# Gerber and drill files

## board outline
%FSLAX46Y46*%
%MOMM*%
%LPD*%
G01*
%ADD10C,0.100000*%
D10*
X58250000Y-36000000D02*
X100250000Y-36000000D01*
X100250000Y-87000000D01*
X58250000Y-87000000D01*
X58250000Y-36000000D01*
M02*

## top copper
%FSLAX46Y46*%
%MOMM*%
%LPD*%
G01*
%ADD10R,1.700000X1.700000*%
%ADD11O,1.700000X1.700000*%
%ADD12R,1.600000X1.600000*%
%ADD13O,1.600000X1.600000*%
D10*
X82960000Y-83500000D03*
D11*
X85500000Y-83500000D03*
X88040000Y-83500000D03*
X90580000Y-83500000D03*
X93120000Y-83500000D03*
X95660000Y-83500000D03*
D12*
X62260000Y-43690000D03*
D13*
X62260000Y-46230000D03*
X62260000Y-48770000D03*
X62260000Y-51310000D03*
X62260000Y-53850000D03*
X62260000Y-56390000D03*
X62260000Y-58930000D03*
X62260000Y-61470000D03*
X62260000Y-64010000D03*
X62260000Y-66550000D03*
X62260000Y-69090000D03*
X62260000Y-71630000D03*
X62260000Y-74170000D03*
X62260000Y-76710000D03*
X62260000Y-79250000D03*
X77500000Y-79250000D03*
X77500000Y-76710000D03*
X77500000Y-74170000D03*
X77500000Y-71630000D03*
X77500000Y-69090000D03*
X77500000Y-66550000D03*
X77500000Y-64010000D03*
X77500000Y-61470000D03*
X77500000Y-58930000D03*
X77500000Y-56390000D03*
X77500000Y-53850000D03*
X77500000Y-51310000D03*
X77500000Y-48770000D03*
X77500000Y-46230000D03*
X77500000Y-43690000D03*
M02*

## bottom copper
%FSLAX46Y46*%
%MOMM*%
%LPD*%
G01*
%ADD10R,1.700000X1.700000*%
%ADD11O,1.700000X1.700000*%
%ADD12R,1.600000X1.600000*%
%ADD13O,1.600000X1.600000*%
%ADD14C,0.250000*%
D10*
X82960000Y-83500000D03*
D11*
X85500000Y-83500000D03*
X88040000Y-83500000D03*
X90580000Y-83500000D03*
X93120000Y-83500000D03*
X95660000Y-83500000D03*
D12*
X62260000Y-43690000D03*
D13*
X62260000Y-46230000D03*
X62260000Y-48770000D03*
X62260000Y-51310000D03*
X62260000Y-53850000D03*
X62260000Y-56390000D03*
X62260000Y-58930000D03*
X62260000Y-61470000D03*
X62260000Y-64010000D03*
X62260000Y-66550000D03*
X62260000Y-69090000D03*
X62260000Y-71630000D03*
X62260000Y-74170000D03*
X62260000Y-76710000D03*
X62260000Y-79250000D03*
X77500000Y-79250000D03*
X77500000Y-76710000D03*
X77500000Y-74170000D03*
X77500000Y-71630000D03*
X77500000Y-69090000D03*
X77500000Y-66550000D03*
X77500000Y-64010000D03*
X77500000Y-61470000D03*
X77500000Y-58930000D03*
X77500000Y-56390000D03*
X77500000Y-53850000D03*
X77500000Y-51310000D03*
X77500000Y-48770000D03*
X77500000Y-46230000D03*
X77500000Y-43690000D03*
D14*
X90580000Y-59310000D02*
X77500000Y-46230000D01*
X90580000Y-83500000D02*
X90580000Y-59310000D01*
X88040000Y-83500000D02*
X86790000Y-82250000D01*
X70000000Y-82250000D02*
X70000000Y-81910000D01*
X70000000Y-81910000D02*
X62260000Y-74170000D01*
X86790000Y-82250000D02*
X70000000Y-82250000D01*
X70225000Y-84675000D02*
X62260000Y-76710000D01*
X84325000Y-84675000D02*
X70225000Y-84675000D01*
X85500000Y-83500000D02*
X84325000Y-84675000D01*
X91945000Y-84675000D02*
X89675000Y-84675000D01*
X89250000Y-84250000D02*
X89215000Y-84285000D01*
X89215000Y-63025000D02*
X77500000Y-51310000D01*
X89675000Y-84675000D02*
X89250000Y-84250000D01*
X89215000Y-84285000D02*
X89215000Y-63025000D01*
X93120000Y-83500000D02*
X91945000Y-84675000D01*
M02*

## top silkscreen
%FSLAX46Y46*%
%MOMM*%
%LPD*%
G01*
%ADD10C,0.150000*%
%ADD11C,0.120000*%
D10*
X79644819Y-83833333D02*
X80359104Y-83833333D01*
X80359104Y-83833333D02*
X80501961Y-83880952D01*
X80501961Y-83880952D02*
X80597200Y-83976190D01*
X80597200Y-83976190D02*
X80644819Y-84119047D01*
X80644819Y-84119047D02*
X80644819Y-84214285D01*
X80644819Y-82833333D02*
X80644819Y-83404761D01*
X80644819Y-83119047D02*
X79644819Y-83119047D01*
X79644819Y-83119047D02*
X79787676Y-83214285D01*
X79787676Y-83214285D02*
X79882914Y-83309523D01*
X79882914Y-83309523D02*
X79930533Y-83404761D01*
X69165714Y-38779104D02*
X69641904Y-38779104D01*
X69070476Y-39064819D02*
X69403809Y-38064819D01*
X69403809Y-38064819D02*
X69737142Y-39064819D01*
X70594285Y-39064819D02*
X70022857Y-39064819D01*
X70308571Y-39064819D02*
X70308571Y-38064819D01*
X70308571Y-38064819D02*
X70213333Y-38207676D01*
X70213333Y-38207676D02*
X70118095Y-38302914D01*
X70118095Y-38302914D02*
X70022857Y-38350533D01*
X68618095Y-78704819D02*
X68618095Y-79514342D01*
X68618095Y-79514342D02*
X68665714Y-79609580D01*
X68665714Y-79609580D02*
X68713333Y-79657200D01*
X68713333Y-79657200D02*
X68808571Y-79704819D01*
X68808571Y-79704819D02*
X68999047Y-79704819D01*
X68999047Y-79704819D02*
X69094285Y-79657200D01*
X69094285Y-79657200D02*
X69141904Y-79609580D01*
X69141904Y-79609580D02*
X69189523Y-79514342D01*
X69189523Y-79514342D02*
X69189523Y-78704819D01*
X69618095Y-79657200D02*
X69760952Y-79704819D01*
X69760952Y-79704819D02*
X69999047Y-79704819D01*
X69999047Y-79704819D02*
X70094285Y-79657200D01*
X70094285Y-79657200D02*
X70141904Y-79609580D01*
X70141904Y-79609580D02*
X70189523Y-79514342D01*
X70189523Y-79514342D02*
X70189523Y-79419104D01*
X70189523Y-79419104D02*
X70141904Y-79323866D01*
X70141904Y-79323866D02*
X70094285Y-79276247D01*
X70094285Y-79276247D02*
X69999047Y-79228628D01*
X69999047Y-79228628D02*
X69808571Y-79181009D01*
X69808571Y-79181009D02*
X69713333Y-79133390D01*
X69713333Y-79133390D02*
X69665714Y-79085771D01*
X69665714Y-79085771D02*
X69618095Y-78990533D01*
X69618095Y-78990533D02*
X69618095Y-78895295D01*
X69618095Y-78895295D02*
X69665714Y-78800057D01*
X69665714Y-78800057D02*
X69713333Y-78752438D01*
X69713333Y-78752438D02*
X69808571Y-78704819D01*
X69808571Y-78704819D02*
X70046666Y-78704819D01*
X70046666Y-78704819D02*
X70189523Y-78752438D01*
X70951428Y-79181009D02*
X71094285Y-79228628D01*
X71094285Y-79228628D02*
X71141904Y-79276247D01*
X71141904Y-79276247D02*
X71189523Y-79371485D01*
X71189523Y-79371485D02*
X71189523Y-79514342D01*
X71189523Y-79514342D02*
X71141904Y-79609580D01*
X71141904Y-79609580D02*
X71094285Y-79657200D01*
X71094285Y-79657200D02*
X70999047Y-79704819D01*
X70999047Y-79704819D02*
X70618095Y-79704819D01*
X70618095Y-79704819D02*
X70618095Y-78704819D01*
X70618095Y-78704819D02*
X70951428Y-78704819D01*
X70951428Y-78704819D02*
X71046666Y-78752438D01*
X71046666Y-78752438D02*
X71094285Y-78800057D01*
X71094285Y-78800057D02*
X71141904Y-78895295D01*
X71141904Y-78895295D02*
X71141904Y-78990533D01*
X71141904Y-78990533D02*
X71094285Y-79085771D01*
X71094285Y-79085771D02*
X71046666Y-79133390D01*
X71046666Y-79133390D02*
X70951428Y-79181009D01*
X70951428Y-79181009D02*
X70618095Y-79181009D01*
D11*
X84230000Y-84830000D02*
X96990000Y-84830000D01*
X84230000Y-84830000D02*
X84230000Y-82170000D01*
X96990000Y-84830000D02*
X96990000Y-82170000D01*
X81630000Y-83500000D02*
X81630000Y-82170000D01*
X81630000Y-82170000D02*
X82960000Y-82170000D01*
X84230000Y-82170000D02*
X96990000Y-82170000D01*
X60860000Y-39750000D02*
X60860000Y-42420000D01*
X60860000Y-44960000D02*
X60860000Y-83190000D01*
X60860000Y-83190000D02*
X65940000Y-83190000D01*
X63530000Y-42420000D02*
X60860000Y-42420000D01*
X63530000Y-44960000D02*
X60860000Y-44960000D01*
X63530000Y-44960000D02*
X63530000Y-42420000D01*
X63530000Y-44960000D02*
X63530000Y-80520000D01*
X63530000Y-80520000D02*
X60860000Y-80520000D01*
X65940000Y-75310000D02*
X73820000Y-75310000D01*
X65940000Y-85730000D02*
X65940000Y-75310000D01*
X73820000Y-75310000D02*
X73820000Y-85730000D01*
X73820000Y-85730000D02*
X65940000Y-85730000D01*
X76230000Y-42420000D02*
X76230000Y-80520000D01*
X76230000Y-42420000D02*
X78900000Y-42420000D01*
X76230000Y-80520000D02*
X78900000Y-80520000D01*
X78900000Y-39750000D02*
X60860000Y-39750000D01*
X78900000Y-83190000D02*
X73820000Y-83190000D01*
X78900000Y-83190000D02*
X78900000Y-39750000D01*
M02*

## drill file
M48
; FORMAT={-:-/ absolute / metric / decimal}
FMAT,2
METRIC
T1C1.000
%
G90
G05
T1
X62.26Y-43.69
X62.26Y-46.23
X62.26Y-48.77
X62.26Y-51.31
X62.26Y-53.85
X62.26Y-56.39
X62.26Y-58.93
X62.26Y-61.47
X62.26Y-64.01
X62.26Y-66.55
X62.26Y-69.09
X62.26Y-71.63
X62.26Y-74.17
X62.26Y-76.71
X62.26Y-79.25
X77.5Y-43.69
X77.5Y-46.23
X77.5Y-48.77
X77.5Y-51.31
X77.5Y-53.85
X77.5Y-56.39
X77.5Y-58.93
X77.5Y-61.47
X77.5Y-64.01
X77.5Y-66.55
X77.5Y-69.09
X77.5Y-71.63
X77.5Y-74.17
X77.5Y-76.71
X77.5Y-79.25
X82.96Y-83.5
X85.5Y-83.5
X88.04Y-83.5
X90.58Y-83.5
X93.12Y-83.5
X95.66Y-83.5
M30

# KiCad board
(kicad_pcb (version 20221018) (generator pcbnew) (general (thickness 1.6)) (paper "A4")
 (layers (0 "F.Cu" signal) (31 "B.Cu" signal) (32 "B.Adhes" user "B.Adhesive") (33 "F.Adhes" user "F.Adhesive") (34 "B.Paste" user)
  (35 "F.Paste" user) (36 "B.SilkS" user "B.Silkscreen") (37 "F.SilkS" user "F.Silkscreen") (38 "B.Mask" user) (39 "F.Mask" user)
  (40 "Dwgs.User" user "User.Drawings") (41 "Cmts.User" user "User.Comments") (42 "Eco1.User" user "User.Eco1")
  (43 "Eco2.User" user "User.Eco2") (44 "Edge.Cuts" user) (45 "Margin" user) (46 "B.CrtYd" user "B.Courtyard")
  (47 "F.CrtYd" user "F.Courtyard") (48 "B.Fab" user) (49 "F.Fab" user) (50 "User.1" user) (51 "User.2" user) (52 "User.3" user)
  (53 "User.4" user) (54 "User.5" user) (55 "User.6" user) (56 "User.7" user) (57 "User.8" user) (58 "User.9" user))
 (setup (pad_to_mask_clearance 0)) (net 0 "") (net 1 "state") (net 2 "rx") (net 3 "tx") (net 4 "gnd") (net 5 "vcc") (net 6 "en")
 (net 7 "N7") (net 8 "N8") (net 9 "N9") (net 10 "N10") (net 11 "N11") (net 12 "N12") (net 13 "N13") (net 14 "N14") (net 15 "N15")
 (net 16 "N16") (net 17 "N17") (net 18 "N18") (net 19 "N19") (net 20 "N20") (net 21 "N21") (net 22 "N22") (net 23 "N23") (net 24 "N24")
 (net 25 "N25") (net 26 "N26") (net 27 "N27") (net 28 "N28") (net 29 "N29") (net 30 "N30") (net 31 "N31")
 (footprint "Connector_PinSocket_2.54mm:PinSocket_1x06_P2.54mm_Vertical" (layer "F.Cu") (at 82.96 83.5 90)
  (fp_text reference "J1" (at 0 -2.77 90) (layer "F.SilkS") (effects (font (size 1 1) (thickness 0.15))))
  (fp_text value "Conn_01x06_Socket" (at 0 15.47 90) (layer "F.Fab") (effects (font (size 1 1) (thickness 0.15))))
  (fp_line (start -1.33 1.27) (end -1.33 14.03) (stroke (width 0.12) (type solid)) (layer "F.SilkS"))
  (fp_line (start -1.33 1.27) (end 1.33 1.27) (stroke (width 0.12) (type solid)) (layer "F.SilkS"))
  (fp_line (start -1.33 14.03) (end 1.33 14.03) (stroke (width 0.12) (type solid)) (layer "F.SilkS"))
  (fp_line (start 0 -1.33) (end 1.33 -1.33) (stroke (width 0.12) (type solid)) (layer "F.SilkS"))
  (fp_line (start 1.33 -1.33) (end 1.33 0) (stroke (width 0.12) (type solid)) (layer "F.SilkS"))
  (fp_line (start 1.33 1.27) (end 1.33 14.03) (stroke (width 0.12) (type solid)) (layer "F.SilkS"))
  (pad "1" thru_hole rect (at 0 0 90) (size 1.7 1.7) (drill 1) (layers "*.Cu" "*.Mask") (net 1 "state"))
  (pad "2" thru_hole oval (at 0 2.54 90) (size 1.7 1.7) (drill 1) (layers "*.Cu" "*.Mask") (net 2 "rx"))
  (pad "3" thru_hole oval (at 0 5.08 90) (size 1.7 1.7) (drill 1) (layers "*.Cu" "*.Mask") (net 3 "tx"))
  (pad "4" thru_hole oval (at 0 7.62 90) (size 1.7 1.7) (drill 1) (layers "*.Cu" "*.Mask") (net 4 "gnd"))
  (pad "5" thru_hole oval (at 0 10.16 90) (size 1.7 1.7) (drill 1) (layers "*.Cu" "*.Mask") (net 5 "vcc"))
  (pad "6" thru_hole oval (at 0 12.7 90) (size 1.7 1.7) (drill 1) (layers "*.Cu" "*.Mask") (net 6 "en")))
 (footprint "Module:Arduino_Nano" (layer "F.Cu") (at 62.26 43.69)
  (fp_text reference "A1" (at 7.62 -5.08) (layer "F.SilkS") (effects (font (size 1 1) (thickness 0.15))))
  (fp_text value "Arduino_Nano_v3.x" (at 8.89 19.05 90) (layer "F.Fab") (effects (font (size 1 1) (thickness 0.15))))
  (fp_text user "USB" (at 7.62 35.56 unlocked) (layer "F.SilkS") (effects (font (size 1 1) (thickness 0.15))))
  (fp_line (start -1.4 -3.94) (end -1.4 -1.27) (stroke (width 0.12) (type solid)) (layer "F.SilkS"))
  (fp_line (start -1.4 1.27) (end -1.4 39.5) (stroke (width 0.12) (type solid)) (layer "F.SilkS"))
  (fp_line (start -1.4 39.5) (end 3.68 39.5) (stroke (width 0.12) (type solid)) (layer "F.SilkS"))
  (fp_line (start 1.27 -1.27) (end -1.4 -1.27) (stroke (width 0.12) (type solid)) (layer "F.SilkS"))
  (fp_line (start 1.27 1.27) (end -1.4 1.27) (stroke (width 0.12) (type solid)) (layer "F.SilkS"))
  (fp_line (start 1.27 1.27) (end 1.27 -1.27) (stroke (width 0.12) (type solid)) (layer "F.SilkS"))
  (fp_line (start 1.27 1.27) (end 1.27 36.83) (stroke (width 0.12) (type solid)) (layer "F.SilkS"))
  (fp_line (start 1.27 36.83) (end -1.4 36.83) (stroke (width 0.12) (type solid)) (layer "F.SilkS"))
  (fp_line (start 3.68 31.62) (end 11.56 31.62) (stroke (width 0.12) (type solid)) (layer "F.SilkS"))
  (fp_line (start 3.68 42.04) (end 3.68 31.62) (stroke (width 0.12) (type solid)) (layer "F.SilkS"))
  (fp_line (start 11.56 31.62) (end 11.56 42.04) (stroke (width 0.12) (type solid)) (layer "F.SilkS"))
  (fp_line (start 11.56 42.04) (end 3.68 42.04) (stroke (width 0.12) (type solid)) (layer "F.SilkS"))
  (fp_line (start 13.97 -1.27) (end 13.97 36.83) (stroke (width 0.12) (type solid)) (layer "F.SilkS"))
  (fp_line (start 13.97 -1.27) (end 16.64 -1.27) (stroke (width 0.12) (type solid)) (layer "F.SilkS"))
  (fp_line (start 13.97 36.83) (end 16.64 36.83) (stroke (width 0.12) (type solid)) (layer "F.SilkS"))
  (fp_line (start 16.64 -3.94) (end -1.4 -3.94) (stroke (width 0.12) (type solid)) (layer "F.SilkS"))
  (fp_line (start 16.64 39.5) (end 11.56 39.5) (stroke (width 0.12) (type solid)) (layer "F.SilkS"))
  (fp_line (start 16.64 39.5) (end 16.64 -3.94) (stroke (width 0.12) (type solid)) (layer "F.SilkS"))
  (pad "1" thru_hole rect (at 0 0) (size 1.6 1.6) (drill 1) (layers "*.Cu" "*.Mask") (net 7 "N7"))
  (pad "2" thru_hole oval (at 0 2.54) (size 1.6 1.6) (drill 1) (layers "*.Cu" "*.Mask") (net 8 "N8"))
  (pad "3" thru_hole oval (at 0 5.08) (size 1.6 1.6) (drill 1) (layers "*.Cu" "*.Mask") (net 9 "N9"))
  (pad "4" thru_hole oval (at 0 7.62) (size 1.6 1.6) (drill 1) (layers "*.Cu" "*.Mask") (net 4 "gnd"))
  (pad "5" thru_hole oval (at 0 10.16) (size 1.6 1.6) (drill 1) (layers "*.Cu" "*.Mask") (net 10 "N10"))
  (pad "6" thru_hole oval (at 0 12.7) (size 1.6 1.6) (drill 1) (layers "*.Cu" "*.Mask") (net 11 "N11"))
  (pad "7" thru_hole oval (at 0 15.24) (size 1.6 1.6) (drill 1) (layers "*.Cu" "*.Mask") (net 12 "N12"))
  (pad "8" thru_hole oval (at 0 17.78) (size 1.6 1.6) (drill 1) (layers "*.Cu" "*.Mask") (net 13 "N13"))
  (pad "9" thru_hole oval (at 0 20.32) (size 1.6 1.6) (drill 1) (layers "*.Cu" "*.Mask") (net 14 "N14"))
  (pad "10" thru_hole oval (at 0 22.86) (size 1.6 1.6) (drill 1) (layers "*.Cu" "*.Mask") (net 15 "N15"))
  (pad "11" thru_hole oval (at 0 25.4) (size 1.6 1.6) (drill 1) (layers "*.Cu" "*.Mask") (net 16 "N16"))
  (pad "12" thru_hole oval (at 0 27.94) (size 1.6 1.6) (drill 1) (layers "*.Cu" "*.Mask") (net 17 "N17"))
  (pad "13" thru_hole oval (at 0 30.48) (size 1.6 1.6) (drill 1) (layers "*.Cu" "*.Mask") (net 3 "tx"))
  (pad "14" thru_hole oval (at 0 33.02) (size 1.6 1.6) (drill 1) (layers "*.Cu" "*.Mask") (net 2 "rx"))
  (pad "15" thru_hole oval (at 0 35.56) (size 1.6 1.6) (drill 1) (layers "*.Cu" "*.Mask") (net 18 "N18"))
  (pad "16" thru_hole oval (at 15.24 35.56) (size 1.6 1.6) (drill 1) (layers "*.Cu" "*.Mask") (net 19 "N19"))
  (pad "17" thru_hole oval (at 15.24 33.02) (size 1.6 1.6) (drill 1) (layers "*.Cu" "*.Mask") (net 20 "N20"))
  (pad "18" thru_hole oval (at 15.24 30.48) (size 1.6 1.6) (drill 1) (layers "*.Cu" "*.Mask") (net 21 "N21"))
  (pad "19" thru_hole oval (at 15.24 27.94) (size 1.6 1.6) (drill 1) (layers "*.Cu" "*.Mask") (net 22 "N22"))
  (pad "20" thru_hole oval (at 15.24 25.4) (size 1.6 1.6) (drill 1) (layers "*.Cu" "*.Mask") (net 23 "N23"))
  (pad "21" thru_hole oval (at 15.24 22.86) (size 1.6 1.6) (drill 1) (layers "*.Cu" "*.Mask") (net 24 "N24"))
  (pad "22" thru_hole oval (at 15.24 20.32) (size 1.6 1.6) (drill 1) (layers "*.Cu" "*.Mask") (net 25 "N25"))
  (pad "23" thru_hole oval (at 15.24 17.78) (size 1.6 1.6) (drill 1) (layers "*.Cu" "*.Mask") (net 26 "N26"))
  (pad "24" thru_hole oval (at 15.24 15.24) (size 1.6 1.6) (drill 1) (layers "*.Cu" "*.Mask") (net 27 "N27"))
  (pad "25" thru_hole oval (at 15.24 12.7) (size 1.6 1.6) (drill 1) (layers "*.Cu" "*.Mask") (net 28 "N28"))
  (pad "26" thru_hole oval (at 15.24 10.16) (size 1.6 1.6) (drill 1) (layers "*.Cu" "*.Mask") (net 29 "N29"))
  (pad "27" thru_hole oval (at 15.24 7.62) (size 1.6 1.6) (drill 1) (layers "*.Cu" "*.Mask") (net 5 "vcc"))
  (pad "28" thru_hole oval (at 15.24 5.08) (size 1.6 1.6) (drill 1) (layers "*.Cu" "*.Mask") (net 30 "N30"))
  (pad "29" thru_hole oval (at 15.24 2.54) (size 1.6 1.6) (drill 1) (layers "*.Cu" "*.Mask") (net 4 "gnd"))
  (pad "30" thru_hole oval (at 15.24 0) (size 1.6 1.6) (drill 1) (layers "*.Cu" "*.Mask") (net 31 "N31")))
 (gr_rect (start 58.25 36) (end 100.25 87) (stroke (width 0.1) (type default)) (fill none) (layer "Edge.Cuts"))
 (segment (start 90.58 59.31) (end 77.5 46.23) (width 0.25) (layer "B.Cu") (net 4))
 (segment (start 90.58 83.5) (end 90.58 59.31) (width 0.25) (layer "B.Cu") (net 4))
 (segment (start 88.04 83.5) (end 86.79 82.25) (width 0.25) (layer "B.Cu") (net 3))
 (segment (start 70 82.25) (end 70 81.91) (width 0.25) (layer "B.Cu") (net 3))
 (segment (start 70 81.91) (end 62.26 74.17) (width 0.25) (layer "B.Cu") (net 3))
 (segment (start 86.79 82.25) (end 70 82.25) (width 0.25) (layer "B.Cu") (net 3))
 (segment (start 70.225 84.675) (end 62.26 76.71) (width 0.25) (layer "B.Cu") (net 2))
 (segment (start 84.325 84.675) (end 70.225 84.675) (width 0.25) (layer "B.Cu") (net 2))
 (segment (start 85.5 83.5) (end 84.325 84.675) (width 0.25) (layer "B.Cu") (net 2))
 (segment (start 91.945 84.675) (end 89.675 84.675) (width 0.25) (layer "B.Cu") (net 5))
 (segment (start 89.25 84.25) (end 89.215 84.285) (width 0.25) (layer "B.Cu") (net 5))
 (segment (start 89.215 63.025) (end 77.5 51.31) (width 0.25) (layer "B.Cu") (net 5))
 (segment (start 89.675 84.675) (end 89.25 84.25) (width 0.25) (layer "B.Cu") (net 5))
 (segment (start 89.215 84.285) (end 89.215 63.025) (width 0.25) (layer "B.Cu") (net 5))
 (segment (start 93.12 83.5) (end 91.945 84.675) (width 0.25) (layer "B.Cu") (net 5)))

